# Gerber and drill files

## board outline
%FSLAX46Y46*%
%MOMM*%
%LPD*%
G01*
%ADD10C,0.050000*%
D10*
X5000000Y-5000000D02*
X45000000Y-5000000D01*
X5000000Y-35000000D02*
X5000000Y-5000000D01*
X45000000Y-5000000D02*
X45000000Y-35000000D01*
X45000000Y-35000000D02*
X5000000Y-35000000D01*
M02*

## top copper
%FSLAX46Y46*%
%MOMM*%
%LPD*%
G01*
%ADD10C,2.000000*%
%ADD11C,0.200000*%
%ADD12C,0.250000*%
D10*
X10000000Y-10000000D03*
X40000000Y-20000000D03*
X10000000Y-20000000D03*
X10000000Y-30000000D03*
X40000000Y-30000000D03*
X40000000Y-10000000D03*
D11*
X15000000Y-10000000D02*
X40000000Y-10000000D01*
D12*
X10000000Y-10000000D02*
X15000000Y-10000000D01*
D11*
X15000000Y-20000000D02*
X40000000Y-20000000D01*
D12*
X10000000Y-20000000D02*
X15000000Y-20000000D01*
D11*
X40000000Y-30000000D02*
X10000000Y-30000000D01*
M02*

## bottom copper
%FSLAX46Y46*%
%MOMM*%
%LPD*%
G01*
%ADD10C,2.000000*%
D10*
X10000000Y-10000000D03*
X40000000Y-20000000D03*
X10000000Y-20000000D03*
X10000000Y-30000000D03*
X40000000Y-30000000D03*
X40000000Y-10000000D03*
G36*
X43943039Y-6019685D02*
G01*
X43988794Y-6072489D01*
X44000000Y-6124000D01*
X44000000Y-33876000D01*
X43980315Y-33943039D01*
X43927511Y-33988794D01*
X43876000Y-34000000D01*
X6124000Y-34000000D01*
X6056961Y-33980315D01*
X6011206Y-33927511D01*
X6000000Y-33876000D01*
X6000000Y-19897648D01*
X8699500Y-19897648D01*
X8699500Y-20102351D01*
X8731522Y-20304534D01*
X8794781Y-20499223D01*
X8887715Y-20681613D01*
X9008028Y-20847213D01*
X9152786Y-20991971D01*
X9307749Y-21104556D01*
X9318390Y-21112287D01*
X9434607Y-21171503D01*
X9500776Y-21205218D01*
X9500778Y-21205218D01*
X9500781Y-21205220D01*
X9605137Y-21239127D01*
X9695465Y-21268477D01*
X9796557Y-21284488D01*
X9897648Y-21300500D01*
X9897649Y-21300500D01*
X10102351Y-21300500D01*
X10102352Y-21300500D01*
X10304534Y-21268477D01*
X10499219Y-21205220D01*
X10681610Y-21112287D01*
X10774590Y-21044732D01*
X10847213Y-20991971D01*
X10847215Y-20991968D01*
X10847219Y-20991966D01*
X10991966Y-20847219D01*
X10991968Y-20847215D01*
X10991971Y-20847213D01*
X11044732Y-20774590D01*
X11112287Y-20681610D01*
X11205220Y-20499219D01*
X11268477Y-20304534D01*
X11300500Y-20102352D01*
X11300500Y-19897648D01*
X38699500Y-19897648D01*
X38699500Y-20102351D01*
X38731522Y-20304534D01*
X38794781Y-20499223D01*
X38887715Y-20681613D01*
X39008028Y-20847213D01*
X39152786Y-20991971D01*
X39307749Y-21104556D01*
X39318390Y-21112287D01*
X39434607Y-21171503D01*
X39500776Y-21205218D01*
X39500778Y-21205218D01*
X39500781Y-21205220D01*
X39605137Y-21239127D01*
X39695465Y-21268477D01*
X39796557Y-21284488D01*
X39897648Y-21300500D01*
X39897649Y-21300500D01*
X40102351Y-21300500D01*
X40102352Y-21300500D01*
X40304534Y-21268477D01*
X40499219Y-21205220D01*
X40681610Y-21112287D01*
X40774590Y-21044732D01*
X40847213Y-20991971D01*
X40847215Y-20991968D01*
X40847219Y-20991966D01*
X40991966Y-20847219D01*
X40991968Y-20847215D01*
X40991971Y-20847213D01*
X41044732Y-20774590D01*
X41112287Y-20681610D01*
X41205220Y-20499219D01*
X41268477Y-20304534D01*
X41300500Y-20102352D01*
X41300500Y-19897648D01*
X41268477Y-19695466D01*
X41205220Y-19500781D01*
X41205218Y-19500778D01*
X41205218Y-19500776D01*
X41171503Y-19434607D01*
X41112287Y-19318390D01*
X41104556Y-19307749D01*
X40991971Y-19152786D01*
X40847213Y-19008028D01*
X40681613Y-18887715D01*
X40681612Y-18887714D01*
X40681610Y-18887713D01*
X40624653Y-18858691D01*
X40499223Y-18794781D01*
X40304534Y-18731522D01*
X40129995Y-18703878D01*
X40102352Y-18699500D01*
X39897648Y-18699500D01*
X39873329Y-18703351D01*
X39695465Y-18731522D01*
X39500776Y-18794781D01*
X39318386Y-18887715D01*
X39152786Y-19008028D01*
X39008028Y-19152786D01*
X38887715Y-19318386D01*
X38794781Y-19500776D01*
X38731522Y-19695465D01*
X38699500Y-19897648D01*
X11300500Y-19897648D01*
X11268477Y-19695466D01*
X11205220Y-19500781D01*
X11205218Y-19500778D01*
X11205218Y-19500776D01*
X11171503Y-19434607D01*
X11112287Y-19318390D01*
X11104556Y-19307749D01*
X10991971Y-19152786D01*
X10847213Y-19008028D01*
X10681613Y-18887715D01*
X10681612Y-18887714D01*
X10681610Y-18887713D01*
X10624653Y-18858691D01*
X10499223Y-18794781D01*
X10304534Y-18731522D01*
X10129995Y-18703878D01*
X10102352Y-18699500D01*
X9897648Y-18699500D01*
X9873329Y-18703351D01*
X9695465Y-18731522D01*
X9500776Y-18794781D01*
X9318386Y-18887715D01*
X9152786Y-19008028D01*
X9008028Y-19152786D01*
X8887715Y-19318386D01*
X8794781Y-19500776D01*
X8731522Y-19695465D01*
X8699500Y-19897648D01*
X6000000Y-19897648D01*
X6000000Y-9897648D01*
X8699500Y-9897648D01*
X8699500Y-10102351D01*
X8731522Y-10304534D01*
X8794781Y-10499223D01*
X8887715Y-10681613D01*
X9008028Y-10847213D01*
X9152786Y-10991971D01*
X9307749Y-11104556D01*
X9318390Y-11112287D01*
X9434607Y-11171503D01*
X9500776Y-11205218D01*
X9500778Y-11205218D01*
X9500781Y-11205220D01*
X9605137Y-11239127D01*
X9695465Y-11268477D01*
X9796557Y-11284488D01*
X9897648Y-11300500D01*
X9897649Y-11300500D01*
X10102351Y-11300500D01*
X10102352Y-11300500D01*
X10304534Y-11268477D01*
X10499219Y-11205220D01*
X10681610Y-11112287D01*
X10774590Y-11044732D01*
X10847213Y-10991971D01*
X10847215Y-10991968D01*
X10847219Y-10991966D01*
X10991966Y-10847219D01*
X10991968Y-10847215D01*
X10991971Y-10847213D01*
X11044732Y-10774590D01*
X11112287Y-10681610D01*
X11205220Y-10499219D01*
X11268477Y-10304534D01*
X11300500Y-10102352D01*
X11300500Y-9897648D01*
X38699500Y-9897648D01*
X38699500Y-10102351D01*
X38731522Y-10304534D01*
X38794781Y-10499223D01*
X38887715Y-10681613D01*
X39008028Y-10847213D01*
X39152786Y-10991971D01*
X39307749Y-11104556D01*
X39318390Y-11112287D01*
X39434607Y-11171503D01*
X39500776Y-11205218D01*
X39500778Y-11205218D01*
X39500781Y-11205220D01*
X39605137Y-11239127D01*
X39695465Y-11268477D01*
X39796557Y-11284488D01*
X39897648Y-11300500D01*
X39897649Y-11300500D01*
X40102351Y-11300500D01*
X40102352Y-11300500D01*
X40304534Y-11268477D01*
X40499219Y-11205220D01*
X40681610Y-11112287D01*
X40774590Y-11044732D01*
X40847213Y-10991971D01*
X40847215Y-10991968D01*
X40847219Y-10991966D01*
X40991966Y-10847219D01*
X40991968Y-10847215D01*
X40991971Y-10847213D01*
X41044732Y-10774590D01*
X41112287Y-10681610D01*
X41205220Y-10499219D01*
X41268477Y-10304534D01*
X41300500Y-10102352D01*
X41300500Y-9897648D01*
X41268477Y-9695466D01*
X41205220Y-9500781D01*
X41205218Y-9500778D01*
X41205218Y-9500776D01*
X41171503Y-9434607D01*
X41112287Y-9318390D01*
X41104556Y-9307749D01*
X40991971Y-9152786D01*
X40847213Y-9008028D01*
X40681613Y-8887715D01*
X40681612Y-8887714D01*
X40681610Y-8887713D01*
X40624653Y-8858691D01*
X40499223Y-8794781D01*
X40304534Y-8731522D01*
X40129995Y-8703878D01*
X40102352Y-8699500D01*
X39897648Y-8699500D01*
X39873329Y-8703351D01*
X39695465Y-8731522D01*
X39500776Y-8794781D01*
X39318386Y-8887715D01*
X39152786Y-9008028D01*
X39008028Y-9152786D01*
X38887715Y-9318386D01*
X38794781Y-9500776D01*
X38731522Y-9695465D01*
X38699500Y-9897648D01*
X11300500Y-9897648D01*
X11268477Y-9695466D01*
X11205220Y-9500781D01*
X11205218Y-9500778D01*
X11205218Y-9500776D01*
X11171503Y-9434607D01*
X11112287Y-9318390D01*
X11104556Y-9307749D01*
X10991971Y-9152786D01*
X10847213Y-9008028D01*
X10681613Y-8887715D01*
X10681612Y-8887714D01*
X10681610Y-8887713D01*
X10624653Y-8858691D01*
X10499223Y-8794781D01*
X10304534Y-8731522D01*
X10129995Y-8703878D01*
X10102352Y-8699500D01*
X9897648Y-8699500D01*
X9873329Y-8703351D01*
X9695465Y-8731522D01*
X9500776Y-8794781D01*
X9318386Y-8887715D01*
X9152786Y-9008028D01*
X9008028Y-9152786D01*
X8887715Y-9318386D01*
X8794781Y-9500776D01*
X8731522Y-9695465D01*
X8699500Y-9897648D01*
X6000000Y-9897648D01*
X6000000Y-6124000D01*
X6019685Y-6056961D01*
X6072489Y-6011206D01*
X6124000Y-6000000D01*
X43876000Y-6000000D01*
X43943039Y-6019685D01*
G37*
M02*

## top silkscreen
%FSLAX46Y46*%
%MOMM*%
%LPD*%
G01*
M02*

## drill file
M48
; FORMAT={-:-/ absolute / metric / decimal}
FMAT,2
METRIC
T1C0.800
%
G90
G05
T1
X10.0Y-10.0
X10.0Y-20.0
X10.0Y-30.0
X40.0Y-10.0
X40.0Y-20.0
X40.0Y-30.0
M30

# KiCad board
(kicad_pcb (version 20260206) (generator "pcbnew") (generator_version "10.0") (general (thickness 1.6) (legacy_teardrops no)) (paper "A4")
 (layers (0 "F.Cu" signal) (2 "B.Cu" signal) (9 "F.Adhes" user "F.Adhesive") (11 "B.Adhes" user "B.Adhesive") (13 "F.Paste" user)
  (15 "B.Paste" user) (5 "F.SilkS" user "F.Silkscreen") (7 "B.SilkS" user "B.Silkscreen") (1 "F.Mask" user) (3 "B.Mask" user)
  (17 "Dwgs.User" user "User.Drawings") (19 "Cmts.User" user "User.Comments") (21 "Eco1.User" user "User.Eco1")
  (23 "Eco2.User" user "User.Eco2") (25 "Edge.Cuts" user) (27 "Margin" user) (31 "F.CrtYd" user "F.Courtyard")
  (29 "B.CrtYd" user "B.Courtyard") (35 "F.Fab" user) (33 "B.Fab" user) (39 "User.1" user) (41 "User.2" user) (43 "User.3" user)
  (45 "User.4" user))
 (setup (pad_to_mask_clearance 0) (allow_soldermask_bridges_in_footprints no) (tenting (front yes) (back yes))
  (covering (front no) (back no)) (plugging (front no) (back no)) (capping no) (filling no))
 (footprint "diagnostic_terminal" (layer "F.Cu") (at 10 10)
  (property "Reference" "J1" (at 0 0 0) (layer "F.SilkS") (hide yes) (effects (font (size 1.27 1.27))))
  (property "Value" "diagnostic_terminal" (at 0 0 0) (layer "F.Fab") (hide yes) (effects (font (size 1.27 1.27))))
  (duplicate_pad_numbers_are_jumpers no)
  (pad "1" thru_hole circle (at 0 0) (size 2 2) (drill 0.8) (layers "*.Cu") (remove_unused_layers no) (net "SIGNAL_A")))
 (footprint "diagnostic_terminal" (layer "F.Cu") (at 40 20)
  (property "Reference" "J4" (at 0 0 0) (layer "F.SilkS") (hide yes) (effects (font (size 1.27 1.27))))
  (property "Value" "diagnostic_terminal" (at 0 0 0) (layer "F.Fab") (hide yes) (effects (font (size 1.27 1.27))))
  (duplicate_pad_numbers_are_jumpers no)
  (pad "1" thru_hole circle (at 0 0) (size 2 2) (drill 0.8) (layers "*.Cu") (remove_unused_layers no) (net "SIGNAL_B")))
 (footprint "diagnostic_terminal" (layer "F.Cu") (at 10 20)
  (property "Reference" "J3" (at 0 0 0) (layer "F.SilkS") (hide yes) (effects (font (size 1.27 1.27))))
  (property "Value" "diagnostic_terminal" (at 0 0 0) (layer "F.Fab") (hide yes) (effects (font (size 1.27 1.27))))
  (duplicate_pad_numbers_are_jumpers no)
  (pad "1" thru_hole circle (at 0 0) (size 2 2) (drill 0.8) (layers "*.Cu") (remove_unused_layers no) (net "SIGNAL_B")))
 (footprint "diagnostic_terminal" (layer "F.Cu") (at 10 30)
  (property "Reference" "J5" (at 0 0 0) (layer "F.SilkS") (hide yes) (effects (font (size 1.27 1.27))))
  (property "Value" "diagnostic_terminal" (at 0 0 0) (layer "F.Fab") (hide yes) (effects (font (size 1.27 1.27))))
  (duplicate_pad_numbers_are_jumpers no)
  (pad "1" thru_hole circle (at 0 0) (size 2 2) (drill 0.8) (layers "*.Cu") (remove_unused_layers no) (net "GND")))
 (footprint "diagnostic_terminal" (layer "F.Cu") (at 40 30)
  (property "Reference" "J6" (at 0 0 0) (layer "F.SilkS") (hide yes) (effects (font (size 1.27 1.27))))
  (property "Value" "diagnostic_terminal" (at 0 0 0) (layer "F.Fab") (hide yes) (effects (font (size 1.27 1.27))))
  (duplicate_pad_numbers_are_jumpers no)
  (pad "1" thru_hole circle (at 0 0) (size 2 2) (drill 0.8) (layers "*.Cu") (remove_unused_layers no) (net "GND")))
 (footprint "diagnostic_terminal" (layer "F.Cu") (at 40 10)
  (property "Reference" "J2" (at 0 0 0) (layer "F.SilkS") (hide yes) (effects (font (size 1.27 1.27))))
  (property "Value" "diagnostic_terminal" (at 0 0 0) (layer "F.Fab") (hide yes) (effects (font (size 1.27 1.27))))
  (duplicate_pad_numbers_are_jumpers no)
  (pad "1" thru_hole circle (at 0 0) (size 2 2) (drill 0.8) (layers "*.Cu") (remove_unused_layers no) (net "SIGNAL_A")))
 (gr_line (start 5 5) (end 45 5) (stroke (width 0.05) (type default)) (layer "Edge.Cuts"))
 (gr_line (start 5 35) (end 5 5) (stroke (width 0.05) (type default)) (layer "Edge.Cuts"))
 (gr_line (start 45 5) (end 45 35) (stroke (width 0.05) (type default)) (layer "Edge.Cuts"))
 (gr_line (start 45 35) (end 5 35) (stroke (width 0.05) (type default)) (layer "Edge.Cuts"))
 (segment (start 15 10) (end 40 10) (width 0.2) (layer "F.Cu") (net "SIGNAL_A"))
 (segment (start 10 10) (end 15 10) (width 0.25) (layer "F.Cu") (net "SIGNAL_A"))
 (segment (start 15 20) (end 40 20) (width 0.2) (layer "F.Cu") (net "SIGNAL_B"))
 (segment (start 10 20) (end 15 20) (width 0.25) (layer "F.Cu") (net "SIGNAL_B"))
 (segment (start 40 30) (end 10 30) (width 0.2) (layer "F.Cu") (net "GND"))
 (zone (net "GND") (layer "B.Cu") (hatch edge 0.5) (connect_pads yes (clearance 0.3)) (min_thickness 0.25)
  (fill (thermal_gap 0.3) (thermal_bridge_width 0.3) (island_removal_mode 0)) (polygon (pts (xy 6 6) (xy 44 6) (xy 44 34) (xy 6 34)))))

